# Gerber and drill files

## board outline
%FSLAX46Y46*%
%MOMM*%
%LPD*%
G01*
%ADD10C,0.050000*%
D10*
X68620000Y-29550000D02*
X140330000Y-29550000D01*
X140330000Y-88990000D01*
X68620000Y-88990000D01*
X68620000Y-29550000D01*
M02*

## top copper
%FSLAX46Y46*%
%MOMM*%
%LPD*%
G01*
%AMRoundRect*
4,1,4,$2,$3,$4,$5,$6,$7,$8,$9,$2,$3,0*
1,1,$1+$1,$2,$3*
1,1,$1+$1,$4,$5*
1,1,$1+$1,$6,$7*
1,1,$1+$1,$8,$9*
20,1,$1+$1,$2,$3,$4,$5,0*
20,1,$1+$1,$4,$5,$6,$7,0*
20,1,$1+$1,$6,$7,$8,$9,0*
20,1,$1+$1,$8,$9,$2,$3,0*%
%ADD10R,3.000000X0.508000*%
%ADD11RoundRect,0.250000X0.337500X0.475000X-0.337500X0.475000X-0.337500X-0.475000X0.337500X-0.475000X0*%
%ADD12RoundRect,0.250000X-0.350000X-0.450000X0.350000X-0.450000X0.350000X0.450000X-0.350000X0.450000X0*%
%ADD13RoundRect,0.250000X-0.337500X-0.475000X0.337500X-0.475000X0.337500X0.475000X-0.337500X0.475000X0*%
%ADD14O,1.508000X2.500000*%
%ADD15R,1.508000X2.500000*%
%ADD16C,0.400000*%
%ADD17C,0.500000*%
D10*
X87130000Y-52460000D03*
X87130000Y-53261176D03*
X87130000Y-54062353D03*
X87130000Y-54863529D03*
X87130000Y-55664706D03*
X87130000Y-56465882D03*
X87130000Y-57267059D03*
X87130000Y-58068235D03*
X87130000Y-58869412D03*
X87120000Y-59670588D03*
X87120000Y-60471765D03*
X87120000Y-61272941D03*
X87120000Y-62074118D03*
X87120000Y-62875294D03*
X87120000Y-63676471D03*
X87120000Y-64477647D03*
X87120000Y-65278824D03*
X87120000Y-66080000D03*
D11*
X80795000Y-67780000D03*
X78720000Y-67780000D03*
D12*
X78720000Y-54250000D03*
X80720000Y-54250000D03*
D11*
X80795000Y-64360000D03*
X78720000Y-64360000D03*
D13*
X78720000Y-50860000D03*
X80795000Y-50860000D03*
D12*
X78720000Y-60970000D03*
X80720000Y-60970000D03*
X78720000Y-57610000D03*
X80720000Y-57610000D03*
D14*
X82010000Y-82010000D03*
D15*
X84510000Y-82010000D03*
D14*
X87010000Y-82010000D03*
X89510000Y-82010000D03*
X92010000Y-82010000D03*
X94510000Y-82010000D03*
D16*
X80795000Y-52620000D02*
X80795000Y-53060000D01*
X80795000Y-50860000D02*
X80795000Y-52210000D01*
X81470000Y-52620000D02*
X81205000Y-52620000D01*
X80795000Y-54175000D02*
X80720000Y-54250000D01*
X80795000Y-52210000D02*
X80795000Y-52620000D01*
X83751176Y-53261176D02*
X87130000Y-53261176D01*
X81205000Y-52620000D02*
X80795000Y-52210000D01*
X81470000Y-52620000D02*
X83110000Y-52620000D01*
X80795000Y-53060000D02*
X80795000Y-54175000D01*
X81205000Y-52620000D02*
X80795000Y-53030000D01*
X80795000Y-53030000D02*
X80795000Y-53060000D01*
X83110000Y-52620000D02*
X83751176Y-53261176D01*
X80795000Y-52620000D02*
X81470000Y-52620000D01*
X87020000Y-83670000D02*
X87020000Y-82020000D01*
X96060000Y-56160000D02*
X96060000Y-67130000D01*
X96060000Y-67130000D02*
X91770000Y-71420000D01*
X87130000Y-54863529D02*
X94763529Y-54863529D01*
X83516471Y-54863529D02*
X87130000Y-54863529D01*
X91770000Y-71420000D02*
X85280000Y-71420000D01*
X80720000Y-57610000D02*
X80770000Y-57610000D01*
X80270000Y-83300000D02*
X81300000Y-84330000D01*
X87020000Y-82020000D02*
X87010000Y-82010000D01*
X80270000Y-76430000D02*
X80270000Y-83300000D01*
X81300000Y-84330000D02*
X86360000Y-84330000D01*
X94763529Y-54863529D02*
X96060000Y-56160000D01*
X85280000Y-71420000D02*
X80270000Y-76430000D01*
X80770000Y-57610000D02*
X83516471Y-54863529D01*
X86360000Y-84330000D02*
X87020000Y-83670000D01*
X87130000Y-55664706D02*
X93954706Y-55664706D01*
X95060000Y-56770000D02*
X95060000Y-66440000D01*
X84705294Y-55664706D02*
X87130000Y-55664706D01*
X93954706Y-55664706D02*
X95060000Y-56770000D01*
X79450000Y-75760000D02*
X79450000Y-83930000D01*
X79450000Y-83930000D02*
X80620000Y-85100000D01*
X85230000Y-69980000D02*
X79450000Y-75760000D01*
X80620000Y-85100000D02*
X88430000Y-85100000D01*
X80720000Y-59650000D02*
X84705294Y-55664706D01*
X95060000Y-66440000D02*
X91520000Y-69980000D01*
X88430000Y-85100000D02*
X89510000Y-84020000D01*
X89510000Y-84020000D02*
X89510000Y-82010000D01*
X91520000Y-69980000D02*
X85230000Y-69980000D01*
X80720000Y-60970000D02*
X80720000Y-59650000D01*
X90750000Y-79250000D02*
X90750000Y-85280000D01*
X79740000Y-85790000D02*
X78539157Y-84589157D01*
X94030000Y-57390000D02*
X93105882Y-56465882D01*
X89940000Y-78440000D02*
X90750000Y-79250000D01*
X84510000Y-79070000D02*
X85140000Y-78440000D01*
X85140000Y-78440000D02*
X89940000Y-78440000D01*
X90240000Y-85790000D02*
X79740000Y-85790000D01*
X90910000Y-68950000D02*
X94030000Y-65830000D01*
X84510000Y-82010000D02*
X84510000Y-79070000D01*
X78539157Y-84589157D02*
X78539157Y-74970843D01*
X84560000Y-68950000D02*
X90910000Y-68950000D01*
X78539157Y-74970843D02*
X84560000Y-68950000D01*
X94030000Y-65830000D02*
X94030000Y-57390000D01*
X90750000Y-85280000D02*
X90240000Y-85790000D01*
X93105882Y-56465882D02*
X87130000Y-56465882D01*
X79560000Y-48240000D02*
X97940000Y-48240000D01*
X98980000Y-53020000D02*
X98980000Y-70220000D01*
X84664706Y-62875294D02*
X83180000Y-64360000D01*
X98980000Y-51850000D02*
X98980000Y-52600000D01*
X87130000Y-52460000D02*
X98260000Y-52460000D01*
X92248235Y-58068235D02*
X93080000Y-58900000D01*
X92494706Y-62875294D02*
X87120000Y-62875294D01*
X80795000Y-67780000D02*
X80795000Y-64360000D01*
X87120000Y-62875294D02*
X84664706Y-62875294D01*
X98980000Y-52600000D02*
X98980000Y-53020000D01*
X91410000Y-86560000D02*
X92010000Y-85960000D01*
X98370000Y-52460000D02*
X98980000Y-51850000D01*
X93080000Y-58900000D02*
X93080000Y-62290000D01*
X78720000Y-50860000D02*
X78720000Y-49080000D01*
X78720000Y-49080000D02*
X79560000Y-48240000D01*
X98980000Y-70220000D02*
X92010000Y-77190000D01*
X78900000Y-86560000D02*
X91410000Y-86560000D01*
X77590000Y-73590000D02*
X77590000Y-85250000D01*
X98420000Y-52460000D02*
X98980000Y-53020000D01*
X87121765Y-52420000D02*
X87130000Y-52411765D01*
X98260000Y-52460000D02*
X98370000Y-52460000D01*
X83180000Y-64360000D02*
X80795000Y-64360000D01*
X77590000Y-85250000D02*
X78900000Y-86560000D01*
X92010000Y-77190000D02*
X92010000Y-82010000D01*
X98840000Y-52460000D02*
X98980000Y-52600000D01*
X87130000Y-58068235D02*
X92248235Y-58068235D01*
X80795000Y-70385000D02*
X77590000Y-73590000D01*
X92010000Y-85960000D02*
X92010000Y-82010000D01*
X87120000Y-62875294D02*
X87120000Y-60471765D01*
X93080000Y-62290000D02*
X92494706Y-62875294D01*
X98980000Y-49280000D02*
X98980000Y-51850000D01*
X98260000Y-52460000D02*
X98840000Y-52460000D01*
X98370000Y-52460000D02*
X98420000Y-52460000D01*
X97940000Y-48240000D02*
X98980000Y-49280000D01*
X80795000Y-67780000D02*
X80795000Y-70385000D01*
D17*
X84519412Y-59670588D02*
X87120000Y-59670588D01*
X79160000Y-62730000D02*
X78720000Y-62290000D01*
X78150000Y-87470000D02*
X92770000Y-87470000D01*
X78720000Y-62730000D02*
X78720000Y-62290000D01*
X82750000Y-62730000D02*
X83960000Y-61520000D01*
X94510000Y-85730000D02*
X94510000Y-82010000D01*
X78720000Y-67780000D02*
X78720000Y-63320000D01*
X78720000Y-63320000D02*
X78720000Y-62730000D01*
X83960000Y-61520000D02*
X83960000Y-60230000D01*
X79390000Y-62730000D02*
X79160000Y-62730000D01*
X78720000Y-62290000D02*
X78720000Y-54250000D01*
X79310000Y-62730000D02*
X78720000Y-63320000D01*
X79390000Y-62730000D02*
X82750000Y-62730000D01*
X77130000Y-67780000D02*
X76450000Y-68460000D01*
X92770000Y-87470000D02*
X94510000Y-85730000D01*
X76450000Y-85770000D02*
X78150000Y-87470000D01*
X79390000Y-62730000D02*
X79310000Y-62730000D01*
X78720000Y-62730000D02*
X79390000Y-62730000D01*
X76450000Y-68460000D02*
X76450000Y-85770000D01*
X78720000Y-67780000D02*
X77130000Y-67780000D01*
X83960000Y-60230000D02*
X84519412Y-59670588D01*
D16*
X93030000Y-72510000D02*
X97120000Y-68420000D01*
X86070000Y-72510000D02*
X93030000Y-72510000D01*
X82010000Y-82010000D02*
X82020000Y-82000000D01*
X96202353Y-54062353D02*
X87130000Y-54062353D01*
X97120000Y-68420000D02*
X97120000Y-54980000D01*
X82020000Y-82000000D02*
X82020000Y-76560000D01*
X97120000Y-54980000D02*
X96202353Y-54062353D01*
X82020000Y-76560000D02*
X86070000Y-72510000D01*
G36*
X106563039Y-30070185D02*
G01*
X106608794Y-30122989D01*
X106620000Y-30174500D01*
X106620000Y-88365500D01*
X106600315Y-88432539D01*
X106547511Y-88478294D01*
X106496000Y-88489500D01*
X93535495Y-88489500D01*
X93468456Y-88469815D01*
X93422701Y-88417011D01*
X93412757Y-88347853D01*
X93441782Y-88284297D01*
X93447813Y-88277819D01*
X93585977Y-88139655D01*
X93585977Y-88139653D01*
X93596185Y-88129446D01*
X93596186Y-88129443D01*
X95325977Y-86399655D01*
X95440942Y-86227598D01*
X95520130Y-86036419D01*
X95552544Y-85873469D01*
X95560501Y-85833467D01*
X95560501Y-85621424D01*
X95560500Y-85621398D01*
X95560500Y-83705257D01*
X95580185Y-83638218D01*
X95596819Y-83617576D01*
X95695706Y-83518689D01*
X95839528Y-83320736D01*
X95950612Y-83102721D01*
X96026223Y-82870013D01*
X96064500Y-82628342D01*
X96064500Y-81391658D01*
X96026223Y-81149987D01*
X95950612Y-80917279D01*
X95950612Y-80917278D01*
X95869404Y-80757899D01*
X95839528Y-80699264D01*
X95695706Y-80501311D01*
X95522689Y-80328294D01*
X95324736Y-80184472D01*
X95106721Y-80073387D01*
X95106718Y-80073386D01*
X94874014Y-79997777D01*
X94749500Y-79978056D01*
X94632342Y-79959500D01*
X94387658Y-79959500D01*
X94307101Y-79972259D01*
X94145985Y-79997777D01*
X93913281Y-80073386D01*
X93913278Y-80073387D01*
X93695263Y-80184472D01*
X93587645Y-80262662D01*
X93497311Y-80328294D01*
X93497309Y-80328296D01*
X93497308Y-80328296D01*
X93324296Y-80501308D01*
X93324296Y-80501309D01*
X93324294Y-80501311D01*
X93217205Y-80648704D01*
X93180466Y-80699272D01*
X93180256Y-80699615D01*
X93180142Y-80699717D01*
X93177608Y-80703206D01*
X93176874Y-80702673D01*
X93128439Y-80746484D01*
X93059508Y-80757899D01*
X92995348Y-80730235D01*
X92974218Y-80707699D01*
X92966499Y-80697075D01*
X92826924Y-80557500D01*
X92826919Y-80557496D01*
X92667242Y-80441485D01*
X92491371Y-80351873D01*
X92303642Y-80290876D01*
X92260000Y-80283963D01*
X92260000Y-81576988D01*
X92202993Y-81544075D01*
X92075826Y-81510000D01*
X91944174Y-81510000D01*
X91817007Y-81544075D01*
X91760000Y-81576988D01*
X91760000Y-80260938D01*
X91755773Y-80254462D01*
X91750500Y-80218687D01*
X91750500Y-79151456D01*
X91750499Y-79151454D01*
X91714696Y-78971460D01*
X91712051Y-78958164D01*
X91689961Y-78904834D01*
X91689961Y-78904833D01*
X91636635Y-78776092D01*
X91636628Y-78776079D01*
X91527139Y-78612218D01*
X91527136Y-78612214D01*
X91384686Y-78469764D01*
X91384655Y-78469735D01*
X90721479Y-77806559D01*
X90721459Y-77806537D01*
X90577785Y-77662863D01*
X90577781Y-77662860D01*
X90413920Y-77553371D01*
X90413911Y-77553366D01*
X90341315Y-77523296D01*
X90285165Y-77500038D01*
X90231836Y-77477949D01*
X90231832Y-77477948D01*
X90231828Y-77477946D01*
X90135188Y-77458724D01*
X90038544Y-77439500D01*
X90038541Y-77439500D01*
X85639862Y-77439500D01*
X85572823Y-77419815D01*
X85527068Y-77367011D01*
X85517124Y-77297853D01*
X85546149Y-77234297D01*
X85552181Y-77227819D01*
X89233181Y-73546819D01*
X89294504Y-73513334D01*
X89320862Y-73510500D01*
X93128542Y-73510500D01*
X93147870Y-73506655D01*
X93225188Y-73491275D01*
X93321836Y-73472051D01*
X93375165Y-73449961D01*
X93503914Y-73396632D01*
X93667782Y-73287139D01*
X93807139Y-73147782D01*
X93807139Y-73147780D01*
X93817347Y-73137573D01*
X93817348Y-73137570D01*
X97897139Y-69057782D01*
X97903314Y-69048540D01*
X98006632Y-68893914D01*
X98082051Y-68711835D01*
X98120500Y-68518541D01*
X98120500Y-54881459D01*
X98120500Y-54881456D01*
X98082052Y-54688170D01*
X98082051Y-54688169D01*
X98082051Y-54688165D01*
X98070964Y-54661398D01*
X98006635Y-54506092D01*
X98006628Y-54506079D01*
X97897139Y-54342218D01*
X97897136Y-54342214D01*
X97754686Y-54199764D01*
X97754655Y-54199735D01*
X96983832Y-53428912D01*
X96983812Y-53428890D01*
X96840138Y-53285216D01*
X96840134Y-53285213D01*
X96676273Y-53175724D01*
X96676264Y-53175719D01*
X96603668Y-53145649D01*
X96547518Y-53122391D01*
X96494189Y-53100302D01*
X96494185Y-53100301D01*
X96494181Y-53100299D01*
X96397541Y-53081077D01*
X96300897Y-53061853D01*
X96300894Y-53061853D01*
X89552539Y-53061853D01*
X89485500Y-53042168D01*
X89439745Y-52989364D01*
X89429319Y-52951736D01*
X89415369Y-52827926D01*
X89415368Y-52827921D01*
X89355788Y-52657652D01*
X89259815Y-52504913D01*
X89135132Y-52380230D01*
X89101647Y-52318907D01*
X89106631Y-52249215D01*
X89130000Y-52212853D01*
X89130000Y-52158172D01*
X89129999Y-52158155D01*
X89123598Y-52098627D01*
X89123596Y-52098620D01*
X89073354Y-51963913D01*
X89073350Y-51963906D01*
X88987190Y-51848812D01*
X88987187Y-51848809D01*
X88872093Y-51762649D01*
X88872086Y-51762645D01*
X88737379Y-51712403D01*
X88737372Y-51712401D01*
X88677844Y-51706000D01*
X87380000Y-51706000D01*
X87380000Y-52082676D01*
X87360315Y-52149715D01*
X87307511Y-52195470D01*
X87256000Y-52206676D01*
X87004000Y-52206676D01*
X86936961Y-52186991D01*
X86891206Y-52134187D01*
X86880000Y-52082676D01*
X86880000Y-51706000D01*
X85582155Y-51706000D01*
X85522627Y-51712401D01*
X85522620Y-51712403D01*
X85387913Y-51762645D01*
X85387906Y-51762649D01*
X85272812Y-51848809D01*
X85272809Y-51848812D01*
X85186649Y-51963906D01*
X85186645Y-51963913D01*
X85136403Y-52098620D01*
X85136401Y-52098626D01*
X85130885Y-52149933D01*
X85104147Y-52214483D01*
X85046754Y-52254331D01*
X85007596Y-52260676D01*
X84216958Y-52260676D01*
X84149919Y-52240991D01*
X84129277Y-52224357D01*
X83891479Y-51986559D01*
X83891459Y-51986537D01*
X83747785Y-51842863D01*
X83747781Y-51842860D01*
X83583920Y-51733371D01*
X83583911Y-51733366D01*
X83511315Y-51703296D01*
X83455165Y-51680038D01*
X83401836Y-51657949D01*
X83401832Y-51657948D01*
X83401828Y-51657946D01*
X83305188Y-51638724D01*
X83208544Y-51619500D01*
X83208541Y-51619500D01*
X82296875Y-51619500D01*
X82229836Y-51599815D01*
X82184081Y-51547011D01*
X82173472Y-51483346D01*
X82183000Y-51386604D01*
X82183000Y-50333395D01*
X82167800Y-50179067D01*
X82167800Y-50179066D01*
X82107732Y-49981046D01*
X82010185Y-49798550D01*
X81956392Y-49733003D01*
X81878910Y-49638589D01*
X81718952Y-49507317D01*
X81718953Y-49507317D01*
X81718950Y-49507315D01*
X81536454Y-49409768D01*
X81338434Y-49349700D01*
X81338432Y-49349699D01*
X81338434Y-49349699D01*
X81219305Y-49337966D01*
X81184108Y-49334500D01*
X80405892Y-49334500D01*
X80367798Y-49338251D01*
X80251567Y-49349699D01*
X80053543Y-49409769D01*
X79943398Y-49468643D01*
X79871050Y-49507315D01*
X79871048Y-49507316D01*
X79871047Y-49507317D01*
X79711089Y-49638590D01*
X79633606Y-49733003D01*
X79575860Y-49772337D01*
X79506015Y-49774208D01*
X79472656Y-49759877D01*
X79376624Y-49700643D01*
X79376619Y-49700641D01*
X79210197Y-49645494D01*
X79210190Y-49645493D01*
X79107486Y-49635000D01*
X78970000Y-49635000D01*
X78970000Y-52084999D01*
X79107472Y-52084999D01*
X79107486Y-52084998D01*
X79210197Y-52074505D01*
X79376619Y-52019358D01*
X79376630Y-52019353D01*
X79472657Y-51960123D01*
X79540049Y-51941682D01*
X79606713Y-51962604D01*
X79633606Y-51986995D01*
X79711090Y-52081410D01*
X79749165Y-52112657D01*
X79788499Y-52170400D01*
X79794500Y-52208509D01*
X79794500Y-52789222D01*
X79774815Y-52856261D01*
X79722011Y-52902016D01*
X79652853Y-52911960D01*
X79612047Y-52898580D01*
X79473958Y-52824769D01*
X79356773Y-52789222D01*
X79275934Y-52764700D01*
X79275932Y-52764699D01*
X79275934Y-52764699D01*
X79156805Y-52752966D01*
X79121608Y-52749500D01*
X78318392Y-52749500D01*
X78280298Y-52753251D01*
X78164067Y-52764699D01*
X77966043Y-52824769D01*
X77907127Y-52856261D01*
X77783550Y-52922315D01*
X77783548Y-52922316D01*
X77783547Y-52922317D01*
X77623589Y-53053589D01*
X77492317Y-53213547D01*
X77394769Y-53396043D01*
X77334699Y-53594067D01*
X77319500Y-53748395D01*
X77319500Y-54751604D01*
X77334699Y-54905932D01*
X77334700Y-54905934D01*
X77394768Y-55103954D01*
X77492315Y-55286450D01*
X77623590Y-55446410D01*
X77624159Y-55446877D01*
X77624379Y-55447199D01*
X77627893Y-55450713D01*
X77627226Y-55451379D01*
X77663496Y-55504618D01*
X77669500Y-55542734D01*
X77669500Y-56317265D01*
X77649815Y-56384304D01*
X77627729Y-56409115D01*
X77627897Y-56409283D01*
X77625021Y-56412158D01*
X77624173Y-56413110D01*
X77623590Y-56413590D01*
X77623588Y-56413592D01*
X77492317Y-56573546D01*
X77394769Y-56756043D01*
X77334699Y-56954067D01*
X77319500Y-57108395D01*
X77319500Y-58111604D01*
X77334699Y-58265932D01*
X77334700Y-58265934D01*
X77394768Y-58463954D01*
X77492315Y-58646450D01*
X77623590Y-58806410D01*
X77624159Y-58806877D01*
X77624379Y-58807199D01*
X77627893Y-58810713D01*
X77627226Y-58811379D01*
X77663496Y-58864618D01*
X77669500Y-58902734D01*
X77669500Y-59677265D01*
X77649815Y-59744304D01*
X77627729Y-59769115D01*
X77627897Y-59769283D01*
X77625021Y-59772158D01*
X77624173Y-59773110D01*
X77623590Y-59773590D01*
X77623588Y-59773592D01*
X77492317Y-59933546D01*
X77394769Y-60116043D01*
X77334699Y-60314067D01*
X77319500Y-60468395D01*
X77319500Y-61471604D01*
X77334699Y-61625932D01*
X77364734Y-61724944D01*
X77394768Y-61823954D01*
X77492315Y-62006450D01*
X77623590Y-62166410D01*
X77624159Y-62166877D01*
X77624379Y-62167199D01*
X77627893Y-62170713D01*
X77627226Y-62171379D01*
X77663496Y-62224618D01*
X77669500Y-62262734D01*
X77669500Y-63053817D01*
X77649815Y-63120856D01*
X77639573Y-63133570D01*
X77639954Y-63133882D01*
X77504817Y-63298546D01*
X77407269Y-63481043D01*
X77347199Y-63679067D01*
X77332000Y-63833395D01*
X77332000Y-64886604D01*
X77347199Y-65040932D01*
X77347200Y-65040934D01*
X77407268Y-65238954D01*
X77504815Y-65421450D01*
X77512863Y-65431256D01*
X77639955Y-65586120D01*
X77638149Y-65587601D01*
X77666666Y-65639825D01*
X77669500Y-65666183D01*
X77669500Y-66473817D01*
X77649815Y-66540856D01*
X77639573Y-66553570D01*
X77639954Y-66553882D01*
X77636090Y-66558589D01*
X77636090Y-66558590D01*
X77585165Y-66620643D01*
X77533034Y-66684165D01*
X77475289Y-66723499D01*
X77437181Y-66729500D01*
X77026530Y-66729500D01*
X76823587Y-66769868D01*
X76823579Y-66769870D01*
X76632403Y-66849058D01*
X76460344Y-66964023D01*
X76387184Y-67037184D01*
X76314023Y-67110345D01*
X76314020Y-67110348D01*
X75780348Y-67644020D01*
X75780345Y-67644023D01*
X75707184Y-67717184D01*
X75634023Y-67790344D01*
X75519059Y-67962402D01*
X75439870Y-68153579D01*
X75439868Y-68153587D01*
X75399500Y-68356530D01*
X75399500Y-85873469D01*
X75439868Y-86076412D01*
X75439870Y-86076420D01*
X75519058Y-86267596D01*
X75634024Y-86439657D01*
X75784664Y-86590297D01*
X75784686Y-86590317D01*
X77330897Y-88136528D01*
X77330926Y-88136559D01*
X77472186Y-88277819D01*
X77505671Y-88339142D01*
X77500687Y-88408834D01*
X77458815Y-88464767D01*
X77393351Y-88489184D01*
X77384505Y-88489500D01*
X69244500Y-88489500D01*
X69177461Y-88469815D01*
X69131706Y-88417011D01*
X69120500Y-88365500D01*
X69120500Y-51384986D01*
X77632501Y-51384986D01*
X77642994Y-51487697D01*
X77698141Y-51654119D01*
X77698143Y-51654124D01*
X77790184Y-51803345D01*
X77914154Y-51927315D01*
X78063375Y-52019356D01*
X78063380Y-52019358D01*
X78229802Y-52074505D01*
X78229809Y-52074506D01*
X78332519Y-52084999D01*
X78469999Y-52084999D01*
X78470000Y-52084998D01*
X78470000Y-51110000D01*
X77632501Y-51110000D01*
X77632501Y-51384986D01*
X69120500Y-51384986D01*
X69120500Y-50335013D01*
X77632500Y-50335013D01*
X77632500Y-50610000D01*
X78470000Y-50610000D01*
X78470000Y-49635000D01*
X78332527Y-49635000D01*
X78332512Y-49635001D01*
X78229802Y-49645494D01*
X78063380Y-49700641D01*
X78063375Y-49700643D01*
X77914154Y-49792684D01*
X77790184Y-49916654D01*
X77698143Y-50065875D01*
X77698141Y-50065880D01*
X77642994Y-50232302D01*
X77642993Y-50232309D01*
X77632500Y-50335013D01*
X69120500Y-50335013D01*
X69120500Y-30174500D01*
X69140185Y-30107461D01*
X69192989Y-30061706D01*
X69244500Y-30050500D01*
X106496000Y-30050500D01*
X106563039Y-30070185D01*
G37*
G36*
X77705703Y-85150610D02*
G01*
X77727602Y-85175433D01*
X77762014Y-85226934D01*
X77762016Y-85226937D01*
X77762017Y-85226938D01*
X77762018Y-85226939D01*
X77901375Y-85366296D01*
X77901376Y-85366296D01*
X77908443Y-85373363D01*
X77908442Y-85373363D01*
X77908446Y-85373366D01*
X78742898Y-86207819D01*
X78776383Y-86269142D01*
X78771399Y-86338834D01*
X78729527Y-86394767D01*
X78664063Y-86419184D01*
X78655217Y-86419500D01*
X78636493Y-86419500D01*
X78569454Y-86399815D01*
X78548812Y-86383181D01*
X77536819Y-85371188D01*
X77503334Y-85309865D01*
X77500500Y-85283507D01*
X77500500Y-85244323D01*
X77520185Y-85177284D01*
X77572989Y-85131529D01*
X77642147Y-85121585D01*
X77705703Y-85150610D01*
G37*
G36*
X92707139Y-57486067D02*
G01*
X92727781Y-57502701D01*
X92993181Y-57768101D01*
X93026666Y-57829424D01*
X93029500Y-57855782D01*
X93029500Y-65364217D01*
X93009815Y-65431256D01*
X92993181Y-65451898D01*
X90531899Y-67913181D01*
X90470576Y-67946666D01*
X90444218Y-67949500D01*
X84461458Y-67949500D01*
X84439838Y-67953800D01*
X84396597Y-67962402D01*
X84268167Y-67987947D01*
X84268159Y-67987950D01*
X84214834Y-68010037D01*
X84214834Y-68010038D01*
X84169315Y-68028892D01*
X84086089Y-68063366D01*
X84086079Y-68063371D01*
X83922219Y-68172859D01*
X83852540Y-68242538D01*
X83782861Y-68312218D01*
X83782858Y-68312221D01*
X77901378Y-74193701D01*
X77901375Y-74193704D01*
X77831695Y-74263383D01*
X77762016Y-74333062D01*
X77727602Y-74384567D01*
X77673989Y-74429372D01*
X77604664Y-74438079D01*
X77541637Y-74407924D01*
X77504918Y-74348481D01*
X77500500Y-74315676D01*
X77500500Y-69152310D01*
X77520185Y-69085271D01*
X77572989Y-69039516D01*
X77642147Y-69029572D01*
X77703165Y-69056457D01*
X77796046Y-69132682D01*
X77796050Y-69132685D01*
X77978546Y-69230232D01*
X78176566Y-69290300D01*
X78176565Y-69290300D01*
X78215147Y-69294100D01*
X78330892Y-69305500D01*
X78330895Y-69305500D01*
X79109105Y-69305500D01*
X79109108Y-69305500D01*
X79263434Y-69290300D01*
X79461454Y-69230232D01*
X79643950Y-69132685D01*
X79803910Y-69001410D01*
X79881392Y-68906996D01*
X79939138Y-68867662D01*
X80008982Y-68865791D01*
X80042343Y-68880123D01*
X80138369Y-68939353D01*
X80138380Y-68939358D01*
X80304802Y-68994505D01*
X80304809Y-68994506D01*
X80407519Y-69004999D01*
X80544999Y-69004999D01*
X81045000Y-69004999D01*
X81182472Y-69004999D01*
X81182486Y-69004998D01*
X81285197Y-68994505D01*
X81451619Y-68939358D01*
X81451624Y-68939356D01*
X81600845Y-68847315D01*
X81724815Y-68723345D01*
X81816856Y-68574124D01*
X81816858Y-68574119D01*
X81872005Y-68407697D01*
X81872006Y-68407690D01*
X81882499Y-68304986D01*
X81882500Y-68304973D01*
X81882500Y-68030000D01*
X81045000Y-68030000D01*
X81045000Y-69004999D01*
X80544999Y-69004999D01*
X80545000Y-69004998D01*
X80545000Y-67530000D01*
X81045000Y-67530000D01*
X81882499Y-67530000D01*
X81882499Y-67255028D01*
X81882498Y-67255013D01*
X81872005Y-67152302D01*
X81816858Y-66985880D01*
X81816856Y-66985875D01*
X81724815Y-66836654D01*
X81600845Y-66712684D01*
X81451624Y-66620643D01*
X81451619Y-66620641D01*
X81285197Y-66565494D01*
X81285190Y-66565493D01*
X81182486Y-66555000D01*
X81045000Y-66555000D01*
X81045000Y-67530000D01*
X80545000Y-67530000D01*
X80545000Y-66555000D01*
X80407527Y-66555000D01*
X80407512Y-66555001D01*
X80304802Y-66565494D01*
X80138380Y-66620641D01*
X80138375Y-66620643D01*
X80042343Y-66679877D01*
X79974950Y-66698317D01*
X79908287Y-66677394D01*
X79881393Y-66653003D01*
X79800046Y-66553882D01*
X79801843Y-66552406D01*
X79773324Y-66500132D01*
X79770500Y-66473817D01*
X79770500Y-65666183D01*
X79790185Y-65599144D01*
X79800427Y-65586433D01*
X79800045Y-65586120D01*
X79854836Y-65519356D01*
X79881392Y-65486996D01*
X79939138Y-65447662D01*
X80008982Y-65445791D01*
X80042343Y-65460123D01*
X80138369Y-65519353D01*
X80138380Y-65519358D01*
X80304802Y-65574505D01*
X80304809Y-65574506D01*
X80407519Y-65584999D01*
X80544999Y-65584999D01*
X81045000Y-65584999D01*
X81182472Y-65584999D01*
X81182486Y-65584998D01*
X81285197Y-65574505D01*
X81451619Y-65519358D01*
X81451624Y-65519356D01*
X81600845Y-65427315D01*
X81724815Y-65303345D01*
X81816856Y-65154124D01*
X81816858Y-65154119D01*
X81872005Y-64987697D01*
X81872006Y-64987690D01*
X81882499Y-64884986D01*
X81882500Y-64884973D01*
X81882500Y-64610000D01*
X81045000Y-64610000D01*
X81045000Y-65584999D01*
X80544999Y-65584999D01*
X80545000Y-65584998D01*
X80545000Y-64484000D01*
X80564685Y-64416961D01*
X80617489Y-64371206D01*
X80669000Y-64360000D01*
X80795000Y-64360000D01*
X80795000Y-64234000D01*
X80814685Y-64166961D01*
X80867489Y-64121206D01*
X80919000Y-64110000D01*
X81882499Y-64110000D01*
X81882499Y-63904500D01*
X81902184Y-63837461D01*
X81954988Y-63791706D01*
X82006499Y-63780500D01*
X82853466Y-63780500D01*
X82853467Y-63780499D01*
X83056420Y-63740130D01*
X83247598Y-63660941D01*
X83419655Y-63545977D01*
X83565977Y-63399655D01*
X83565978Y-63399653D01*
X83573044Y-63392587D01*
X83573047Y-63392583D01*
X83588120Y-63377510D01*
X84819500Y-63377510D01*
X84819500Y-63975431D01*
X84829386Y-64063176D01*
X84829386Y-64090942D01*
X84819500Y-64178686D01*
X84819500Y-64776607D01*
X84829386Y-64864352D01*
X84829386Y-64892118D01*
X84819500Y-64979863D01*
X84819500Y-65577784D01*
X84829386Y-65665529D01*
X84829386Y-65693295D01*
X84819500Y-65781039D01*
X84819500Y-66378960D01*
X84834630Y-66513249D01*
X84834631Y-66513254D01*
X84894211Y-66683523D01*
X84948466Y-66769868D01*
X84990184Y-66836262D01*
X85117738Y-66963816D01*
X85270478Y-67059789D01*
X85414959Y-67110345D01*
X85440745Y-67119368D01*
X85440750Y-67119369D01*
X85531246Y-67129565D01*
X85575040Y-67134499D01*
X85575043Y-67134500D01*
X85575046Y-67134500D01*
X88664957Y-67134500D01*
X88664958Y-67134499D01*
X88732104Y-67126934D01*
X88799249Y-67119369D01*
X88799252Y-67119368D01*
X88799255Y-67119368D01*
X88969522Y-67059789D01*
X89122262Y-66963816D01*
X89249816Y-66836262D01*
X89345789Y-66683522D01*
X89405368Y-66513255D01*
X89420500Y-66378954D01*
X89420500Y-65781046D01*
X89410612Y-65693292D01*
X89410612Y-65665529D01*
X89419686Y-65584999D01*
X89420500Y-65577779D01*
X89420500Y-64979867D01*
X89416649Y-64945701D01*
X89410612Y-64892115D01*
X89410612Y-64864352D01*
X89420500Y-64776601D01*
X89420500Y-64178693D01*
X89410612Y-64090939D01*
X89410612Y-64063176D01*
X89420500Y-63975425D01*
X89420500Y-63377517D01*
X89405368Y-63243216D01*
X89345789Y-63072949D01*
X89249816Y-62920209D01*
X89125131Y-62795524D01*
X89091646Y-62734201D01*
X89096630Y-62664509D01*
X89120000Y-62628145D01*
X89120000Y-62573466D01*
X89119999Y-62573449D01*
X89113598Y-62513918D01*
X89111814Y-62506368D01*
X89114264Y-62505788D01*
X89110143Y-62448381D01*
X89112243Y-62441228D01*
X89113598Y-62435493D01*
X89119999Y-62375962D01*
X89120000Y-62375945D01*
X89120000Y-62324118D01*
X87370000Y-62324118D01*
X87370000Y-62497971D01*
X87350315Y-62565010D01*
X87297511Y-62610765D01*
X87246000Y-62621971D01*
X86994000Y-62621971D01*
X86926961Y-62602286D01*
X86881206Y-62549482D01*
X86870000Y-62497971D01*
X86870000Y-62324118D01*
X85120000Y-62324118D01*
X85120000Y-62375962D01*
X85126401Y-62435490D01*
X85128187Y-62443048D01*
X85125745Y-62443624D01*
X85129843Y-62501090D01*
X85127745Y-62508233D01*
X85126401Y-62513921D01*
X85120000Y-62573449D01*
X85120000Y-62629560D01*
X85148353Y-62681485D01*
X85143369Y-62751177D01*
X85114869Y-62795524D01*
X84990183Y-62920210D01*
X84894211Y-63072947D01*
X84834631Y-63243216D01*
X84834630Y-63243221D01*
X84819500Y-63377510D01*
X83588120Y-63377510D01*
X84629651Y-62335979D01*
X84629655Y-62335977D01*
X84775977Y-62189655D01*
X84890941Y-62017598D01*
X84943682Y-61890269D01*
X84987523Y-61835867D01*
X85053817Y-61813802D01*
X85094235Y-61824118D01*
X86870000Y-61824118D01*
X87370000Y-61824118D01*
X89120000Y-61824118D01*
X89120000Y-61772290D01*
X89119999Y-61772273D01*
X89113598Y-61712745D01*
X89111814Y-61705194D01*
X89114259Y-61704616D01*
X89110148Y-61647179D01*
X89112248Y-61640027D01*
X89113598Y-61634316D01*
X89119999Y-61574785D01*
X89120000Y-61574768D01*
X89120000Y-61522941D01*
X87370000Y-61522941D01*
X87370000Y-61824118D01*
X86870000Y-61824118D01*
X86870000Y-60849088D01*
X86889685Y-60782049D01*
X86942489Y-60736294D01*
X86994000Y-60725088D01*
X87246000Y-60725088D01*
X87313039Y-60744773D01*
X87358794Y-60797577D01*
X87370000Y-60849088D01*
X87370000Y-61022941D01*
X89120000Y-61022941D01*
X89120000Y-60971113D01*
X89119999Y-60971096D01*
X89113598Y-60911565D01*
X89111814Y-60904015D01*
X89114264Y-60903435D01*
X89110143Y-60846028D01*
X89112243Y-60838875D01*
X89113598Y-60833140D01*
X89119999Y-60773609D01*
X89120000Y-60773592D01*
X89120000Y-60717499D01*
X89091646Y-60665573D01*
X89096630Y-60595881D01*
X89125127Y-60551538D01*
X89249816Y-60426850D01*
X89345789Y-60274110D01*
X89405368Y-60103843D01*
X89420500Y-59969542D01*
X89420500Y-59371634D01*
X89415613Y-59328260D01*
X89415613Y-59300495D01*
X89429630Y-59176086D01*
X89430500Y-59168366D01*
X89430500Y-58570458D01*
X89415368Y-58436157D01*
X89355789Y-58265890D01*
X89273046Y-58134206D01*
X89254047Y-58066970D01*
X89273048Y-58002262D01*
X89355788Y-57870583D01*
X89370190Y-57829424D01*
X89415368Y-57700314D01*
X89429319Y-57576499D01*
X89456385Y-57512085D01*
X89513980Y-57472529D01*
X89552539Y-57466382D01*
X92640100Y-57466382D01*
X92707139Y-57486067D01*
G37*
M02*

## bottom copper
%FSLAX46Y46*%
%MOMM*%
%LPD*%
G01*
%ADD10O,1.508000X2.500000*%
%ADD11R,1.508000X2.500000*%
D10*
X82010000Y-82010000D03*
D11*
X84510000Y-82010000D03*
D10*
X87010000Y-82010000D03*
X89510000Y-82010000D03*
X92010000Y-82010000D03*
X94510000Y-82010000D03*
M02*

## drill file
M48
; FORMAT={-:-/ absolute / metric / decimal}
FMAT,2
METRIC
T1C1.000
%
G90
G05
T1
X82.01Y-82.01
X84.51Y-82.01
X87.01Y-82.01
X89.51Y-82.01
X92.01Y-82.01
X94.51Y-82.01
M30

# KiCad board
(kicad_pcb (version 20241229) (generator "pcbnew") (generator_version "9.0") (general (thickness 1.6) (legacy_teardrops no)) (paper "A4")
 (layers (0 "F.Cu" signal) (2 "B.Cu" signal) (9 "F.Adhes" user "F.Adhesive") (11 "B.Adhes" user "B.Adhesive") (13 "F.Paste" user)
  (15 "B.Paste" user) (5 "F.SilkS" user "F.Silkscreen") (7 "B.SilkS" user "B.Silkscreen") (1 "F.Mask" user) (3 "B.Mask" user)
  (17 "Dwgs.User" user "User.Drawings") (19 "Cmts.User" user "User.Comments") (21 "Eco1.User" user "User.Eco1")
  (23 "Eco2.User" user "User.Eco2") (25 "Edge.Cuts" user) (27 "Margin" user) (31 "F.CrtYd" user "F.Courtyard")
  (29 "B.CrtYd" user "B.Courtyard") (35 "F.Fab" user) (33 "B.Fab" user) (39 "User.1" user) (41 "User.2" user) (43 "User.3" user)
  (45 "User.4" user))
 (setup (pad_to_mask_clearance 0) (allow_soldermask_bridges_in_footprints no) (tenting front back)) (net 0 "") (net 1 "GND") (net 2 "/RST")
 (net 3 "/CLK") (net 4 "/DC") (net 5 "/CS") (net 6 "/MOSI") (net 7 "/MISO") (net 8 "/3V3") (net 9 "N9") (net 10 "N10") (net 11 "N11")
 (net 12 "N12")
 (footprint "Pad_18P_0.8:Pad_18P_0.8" (layer "F.Cu") (at 83.19 58.381176 -90)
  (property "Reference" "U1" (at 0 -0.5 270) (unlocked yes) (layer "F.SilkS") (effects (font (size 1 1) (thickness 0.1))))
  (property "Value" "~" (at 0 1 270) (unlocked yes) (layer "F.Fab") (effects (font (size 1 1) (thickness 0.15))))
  (pad "01" smd rect (at -5.921176 -3.94 270) (size 0.508 3) (layers "F.Cu" "F.Mask" "F.Paste") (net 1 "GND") (solder_mask_margin 0.102))
  (pad "02" smd rect (at -5.12 -3.94 270) (size 0.508 3) (layers "F.Cu" "F.Mask" "F.Paste") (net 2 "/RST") (solder_mask_margin 0.102))
  (pad "03" smd rect (at -4.318823 -3.94 270) (size 0.508 3) (layers "F.Cu" "F.Mask" "F.Paste") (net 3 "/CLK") (solder_mask_margin 0.102))
  (pad "04" smd rect (at -3.517647 -3.94 270) (size 0.508 3) (layers "F.Cu" "F.Mask" "F.Paste") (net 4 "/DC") (solder_mask_margin 0.102))
  (pad "05" smd rect (at -2.71647 -3.94 270) (size 0.508 3) (layers "F.Cu" "F.Mask" "F.Paste") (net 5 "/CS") (solder_mask_margin 0.102))
  (pad "06" smd rect (at -1.915294 -3.94 270) (size 0.508 3) (layers "F.Cu" "F.Mask" "F.Paste") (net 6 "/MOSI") (solder_mask_margin 0.102))
  (pad "07" smd rect (at -1.114117 -3.94 270) (size 0.508 3) (layers "F.Cu" "F.Mask" "F.Paste") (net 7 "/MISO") (solder_mask_margin 0.102))
  (pad "08" smd rect (at -0.312941 -3.94 270) (size 0.508 3) (layers "F.Cu" "F.Mask" "F.Paste") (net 1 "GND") (solder_mask_margin 0.102))
  (pad "09" smd rect (at 0.488236 -3.94 270) (size 0.508 3) (layers "F.Cu" "F.Mask" "F.Paste") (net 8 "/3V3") (solder_mask_margin 0.102))
  (pad "10" smd rect (at 1.289412 -3.93 270) (size 0.508 3) (layers "F.Cu" "F.Mask" "F.Paste") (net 8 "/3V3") (solder_mask_margin 0.102))
  (pad "11" smd rect (at 2.090589 -3.93 270) (size 0.508 3) (layers "F.Cu" "F.Mask" "F.Paste") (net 1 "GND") (solder_mask_margin 0.102))
  (pad "12" smd rect (at 2.891765 -3.93 270) (size 0.508 3) (layers "F.Cu" "F.Mask" "F.Paste") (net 1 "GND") (solder_mask_margin 0.102))
  (pad "13" smd rect (at 3.692942 -3.93 270) (size 0.508 3) (layers "F.Cu" "F.Mask" "F.Paste") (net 1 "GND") (solder_mask_margin 0.102))
  (pad "14" smd rect (at 4.494118 -3.93 270) (size 0.508 3) (layers "F.Cu" "F.Mask" "F.Paste") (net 1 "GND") (solder_mask_margin 0.102))
  (pad "15" smd rect (at 5.295295 -3.93 270) (size 0.508 3) (layers "F.Cu" "F.Mask" "F.Paste") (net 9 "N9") (solder_mask_margin 0.102))
  (pad "16" smd rect (at 6.096471 -3.93 270) (size 0.508 3) (layers "F.Cu" "F.Mask" "F.Paste") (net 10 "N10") (solder_mask_margin 0.102))
  (pad "17" smd rect (at 6.897648 -3.93 270) (size 0.508 3) (layers "F.Cu" "F.Mask" "F.Paste") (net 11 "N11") (solder_mask_margin 0.102))
  (pad "18" smd rect (at 7.698824 -3.93 270) (size 0.508 3) (layers "F.Cu" "F.Mask" "F.Paste") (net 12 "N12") (solder_mask_margin 0.102)))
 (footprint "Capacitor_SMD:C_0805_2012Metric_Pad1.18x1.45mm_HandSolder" (layer "F.Cu") (at 79.7575 67.78 180)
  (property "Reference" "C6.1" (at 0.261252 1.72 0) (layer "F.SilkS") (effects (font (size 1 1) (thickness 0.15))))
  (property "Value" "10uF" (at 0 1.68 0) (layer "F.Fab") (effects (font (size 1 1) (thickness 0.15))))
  (pad "1" smd roundrect (at -1.0375 0 180) (size 1.175 1.45) (layers "F.Cu" "F.Mask" "F.Paste") (roundrect_rratio 0.212766) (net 1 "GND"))
  (pad "2" smd roundrect (at 1.0375 0 180) (size 1.175 1.45) (layers "F.Cu" "F.Mask" "F.Paste") (roundrect_rratio 0.212766) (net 8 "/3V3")))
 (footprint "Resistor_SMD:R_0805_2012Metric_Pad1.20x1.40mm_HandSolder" (layer "F.Cu") (at 79.72 54.25)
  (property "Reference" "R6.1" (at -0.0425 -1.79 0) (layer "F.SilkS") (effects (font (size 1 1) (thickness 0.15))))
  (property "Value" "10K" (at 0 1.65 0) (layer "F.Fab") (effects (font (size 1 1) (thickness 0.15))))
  (pad "1" smd roundrect (at -1 0) (size 1.2 1.4) (layers "F.Cu" "F.Mask" "F.Paste") (roundrect_rratio 0.208333) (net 8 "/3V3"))
  (pad "2" smd roundrect (at 1 0) (size 1.2 1.4) (layers "F.Cu" "F.Mask" "F.Paste") (roundrect_rratio 0.208333) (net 2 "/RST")))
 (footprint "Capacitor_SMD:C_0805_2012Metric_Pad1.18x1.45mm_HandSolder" (layer "F.Cu") (at 79.7575 64.36 180)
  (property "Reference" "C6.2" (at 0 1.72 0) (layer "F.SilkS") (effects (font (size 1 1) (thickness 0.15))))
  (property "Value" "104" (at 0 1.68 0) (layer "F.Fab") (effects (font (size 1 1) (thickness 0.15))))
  (pad "1" smd roundrect (at -1.0375 0 180) (size 1.175 1.45) (layers "F.Cu" "F.Mask" "F.Paste") (roundrect_rratio 0.212766) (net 1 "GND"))
  (pad "2" smd roundrect (at 1.0375 0 180) (size 1.175 1.45) (layers "F.Cu" "F.Mask" "F.Paste") (roundrect_rratio 0.212766) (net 8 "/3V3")))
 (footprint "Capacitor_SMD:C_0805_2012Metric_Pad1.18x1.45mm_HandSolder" (layer "F.Cu") (at 79.7575 50.86)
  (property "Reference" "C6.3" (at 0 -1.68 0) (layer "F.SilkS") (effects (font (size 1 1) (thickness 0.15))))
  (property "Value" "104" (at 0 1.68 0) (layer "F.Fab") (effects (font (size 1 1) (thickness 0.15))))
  (pad "1" smd roundrect (at -1.0375 0) (size 1.175 1.45) (layers "F.Cu" "F.Mask" "F.Paste") (roundrect_rratio 0.212766) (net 1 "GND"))
  (pad "2" smd roundrect (at 1.0375 0) (size 1.175 1.45) (layers "F.Cu" "F.Mask" "F.Paste") (roundrect_rratio 0.212766) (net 2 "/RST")))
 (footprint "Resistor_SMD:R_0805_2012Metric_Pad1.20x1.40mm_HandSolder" (layer "F.Cu") (at 79.72 60.97)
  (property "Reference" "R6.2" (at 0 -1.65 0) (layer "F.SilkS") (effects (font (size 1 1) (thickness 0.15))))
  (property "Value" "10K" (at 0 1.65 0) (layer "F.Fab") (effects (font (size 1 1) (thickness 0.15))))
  (pad "1" smd roundrect (at -1 0) (size 1.2 1.4) (layers "F.Cu" "F.Mask" "F.Paste") (roundrect_rratio 0.208333) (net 8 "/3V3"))
  (pad "2" smd roundrect (at 1 0) (size 1.2 1.4) (layers "F.Cu" "F.Mask" "F.Paste") (roundrect_rratio 0.208333) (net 5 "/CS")))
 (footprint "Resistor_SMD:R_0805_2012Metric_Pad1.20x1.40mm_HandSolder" (layer "F.Cu") (at 79.72 57.61)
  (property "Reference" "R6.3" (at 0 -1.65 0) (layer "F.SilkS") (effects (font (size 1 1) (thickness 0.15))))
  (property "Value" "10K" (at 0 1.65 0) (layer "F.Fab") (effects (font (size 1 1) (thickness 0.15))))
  (pad "1" smd roundrect (at -1 0) (size 1.2 1.4) (layers "F.Cu" "F.Mask" "F.Paste") (roundrect_rratio 0.208333) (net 8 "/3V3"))
  (pad "2" smd roundrect (at 1 0) (size 1.2 1.4) (layers "F.Cu" "F.Mask" "F.Paste") (roundrect_rratio 0.208333) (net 4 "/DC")))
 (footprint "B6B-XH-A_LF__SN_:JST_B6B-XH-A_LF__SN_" (layer "B.Cu") (at 88.26 81.485 180)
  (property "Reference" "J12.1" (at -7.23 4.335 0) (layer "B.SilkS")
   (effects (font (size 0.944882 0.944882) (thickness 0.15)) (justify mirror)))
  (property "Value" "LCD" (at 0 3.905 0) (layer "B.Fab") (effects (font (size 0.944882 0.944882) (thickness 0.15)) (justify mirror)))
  (pad "1" thru_hole oval (at 6.25 -0.525 180) (size 1.508 2.5) (drill 1) (layers "*.Cu" "*.Mask") (remove_unused_layers no) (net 3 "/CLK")
   (solder_mask_margin 0.102))
  (pad "2" thru_hole rect (at 3.75 -0.525 180) (size 1.508 2.5) (drill 1) (layers "*.Cu" "*.Mask") (remove_unused_layers no) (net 6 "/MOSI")
   (solder_mask_margin 0.102))
  (pad "3" thru_hole oval (at 1.25 -0.525 180) (size 1.508 2.5) (drill 1) (layers "*.Cu" "*.Mask") (remove_unused_layers no) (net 4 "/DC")
   (solder_mask_margin 0.102))
  (pad "4" thru_hole oval (at -1.25 -0.525 180) (size 1.508 2.5) (drill 1) (layers "*.Cu" "*.Mask") (remove_unused_layers no) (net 5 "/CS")
   (solder_mask_margin 0.102))
  (pad "5" thru_hole oval (at -3.75 -0.525 180) (size 1.508 2.5) (drill 1) (layers "*.Cu" "*.Mask") (remove_unused_layers no) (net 1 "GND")
   (solder_mask_margin 0.102))
  (pad "6" thru_hole oval (at -6.25 -0.525 180) (size 1.508 2.5) (drill 1) (layers "*.Cu" "*.Mask") (remove_unused_layers no) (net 8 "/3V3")
   (solder_mask_margin 0.102)))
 (gr_rect (start 68.62 29.55) (end 140.33 88.99) (stroke (width 0.05) (type default)) (fill no) (layer "Edge.Cuts"))
 (segment (start 80.795 52.62) (end 80.795 53.06) (width 0.4) (layer "F.Cu") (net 2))
 (segment (start 80.795 50.86) (end 80.795 52.21) (width 0.4) (layer "F.Cu") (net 2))
 (segment (start 81.47 52.62) (end 81.205 52.62) (width 0.4) (layer "F.Cu") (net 2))
 (segment (start 80.795 54.175) (end 80.72 54.25) (width 0.4) (layer "F.Cu") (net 2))
 (segment (start 80.795 52.21) (end 80.795 52.62) (width 0.4) (layer "F.Cu") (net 2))
 (segment (start 83.751176 53.261176) (end 87.13 53.261176) (width 0.4) (layer "F.Cu") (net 2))
 (segment (start 81.205 52.62) (end 80.795 52.21) (width 0.4) (layer "F.Cu") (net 2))
 (segment (start 81.47 52.62) (end 83.11 52.62) (width 0.4) (layer "F.Cu") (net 2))
 (segment (start 80.795 53.06) (end 80.795 54.175) (width 0.4) (layer "F.Cu") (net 2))
 (segment (start 81.205 52.62) (end 80.795 53.03) (width 0.4) (layer "F.Cu") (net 2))
 (segment (start 80.795 53.03) (end 80.795 53.06) (width 0.4) (layer "F.Cu") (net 2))
 (segment (start 83.11 52.62) (end 83.751176 53.261176) (width 0.4) (layer "F.Cu") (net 2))
 (segment (start 80.795 52.62) (end 81.47 52.62) (width 0.4) (layer "F.Cu") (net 2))
 (segment (start 87.02 83.67) (end 87.02 82.02) (width 0.4) (layer "F.Cu") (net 4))
 (segment (start 96.06 56.16) (end 96.06 67.13) (width 0.4) (layer "F.Cu") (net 4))
 (segment (start 96.06 67.13) (end 91.77 71.42) (width 0.4) (layer "F.Cu") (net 4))
 (segment (start 87.13 54.863529) (end 94.763529 54.863529) (width 0.4) (layer "F.Cu") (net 4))
 (segment (start 83.516471 54.863529) (end 87.13 54.863529) (width 0.4) (layer "F.Cu") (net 4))
 (segment (start 91.77 71.42) (end 85.28 71.42) (width 0.4) (layer "F.Cu") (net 4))
 (segment (start 80.72 57.61) (end 80.77 57.61) (width 0.4) (layer "F.Cu") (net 4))
 (segment (start 80.27 83.3) (end 81.3 84.33) (width 0.4) (layer "F.Cu") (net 4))
 (segment (start 87.02 82.02) (end 87.01 82.01) (width 0.4) (layer "F.Cu") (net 4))
 (segment (start 80.27 76.43) (end 80.27 83.3) (width 0.4) (layer "F.Cu") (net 4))
 (segment (start 81.3 84.33) (end 86.36 84.33) (width 0.4) (layer "F.Cu") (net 4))
 (segment (start 94.763529 54.863529) (end 96.06 56.16) (width 0.4) (layer "F.Cu") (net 4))
 (segment (start 85.28 71.42) (end 80.27 76.43) (width 0.4) (layer "F.Cu") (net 4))
 (segment (start 80.77 57.61) (end 83.516471 54.863529) (width 0.4) (layer "F.Cu") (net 4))
 (segment (start 86.36 84.33) (end 87.02 83.67) (width 0.4) (layer "F.Cu") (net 4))
 (segment (start 87.13 55.664706) (end 93.954706 55.664706) (width 0.4) (layer "F.Cu") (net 5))
 (segment (start 95.06 56.77) (end 95.06 66.44) (width 0.4) (layer "F.Cu") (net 5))
 (segment (start 84.705294 55.664706) (end 87.13 55.664706) (width 0.4) (layer "F.Cu") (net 5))
 (segment (start 93.954706 55.664706) (end 95.06 56.77) (width 0.4) (layer "F.Cu") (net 5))
 (segment (start 79.45 75.76) (end 79.45 83.93) (width 0.4) (layer "F.Cu") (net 5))
 (segment (start 79.45 83.93) (end 80.62 85.1) (width 0.4) (layer "F.Cu") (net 5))
 (segment (start 85.23 69.98) (end 79.45 75.76) (width 0.4) (layer "F.Cu") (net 5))
 (segment (start 80.62 85.1) (end 88.43 85.1) (width 0.4) (layer "F.Cu") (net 5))
 (segment (start 80.72 59.65) (end 84.705294 55.664706) (width 0.4) (layer "F.Cu") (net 5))
 (segment (start 95.06 66.44) (end 91.52 69.98) (width 0.4) (layer "F.Cu") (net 5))
 (segment (start 88.43 85.1) (end 89.51 84.02) (width 0.4) (layer "F.Cu") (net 5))
 (segment (start 89.51 84.02) (end 89.51 82.01) (width 0.4) (layer "F.Cu") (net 5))
 (segment (start 91.52 69.98) (end 85.23 69.98) (width 0.4) (layer "F.Cu") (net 5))
 (segment (start 80.72 60.97) (end 80.72 59.65) (width 0.4) (layer "F.Cu") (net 5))
 (segment (start 90.75 79.25) (end 90.75 85.28) (width 0.4) (layer "F.Cu") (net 6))
 (segment (start 79.74 85.79) (end 78.539157 84.589157) (width 0.4) (layer "F.Cu") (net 6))
 (segment (start 94.03 57.39) (end 93.105882 56.465882) (width 0.4) (layer "F.Cu") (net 6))
 (segment (start 89.94 78.44) (end 90.75 79.25) (width 0.4) (layer "F.Cu") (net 6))
 (segment (start 84.51 79.07) (end 85.14 78.44) (width 0.4) (layer "F.Cu") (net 6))
 (segment (start 85.14 78.44) (end 89.94 78.44) (width 0.4) (layer "F.Cu") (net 6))
 (segment (start 90.24 85.79) (end 79.74 85.79) (width 0.4) (layer "F.Cu") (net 6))
 (segment (start 90.91 68.95) (end 94.03 65.83) (width 0.4) (layer "F.Cu") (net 6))
 (segment (start 84.51 82.01) (end 84.51 79.07) (width 0.4) (layer "F.Cu") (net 6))
 (segment (start 78.539157 84.589157) (end 78.539157 74.970843) (width 0.4) (layer "F.Cu") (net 6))
 (segment (start 84.56 68.95) (end 90.91 68.95) (width 0.4) (layer "F.Cu") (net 6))
 (segment (start 78.539157 74.970843) (end 84.56 68.95) (width 0.4) (layer "F.Cu") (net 6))
 (segment (start 94.03 65.83) (end 94.03 57.39) (width 0.4) (layer "F.Cu") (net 6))
 (segment (start 90.75 85.28) (end 90.24 85.79) (width 0.4) (layer "F.Cu") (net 6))
 (segment (start 93.105882 56.465882) (end 87.13 56.465882) (width 0.4) (layer "F.Cu") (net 6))
 (segment (start 79.56 48.24) (end 97.94 48.24) (width 0.4) (layer "F.Cu") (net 1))
 (segment (start 98.98 53.02) (end 98.98 70.22) (width 0.4) (layer "F.Cu") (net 1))
 (segment (start 84.664706 62.875294) (end 83.18 64.36) (width 0.4) (layer "F.Cu") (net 1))
 (segment (start 98.98 51.85) (end 98.98 52.6) (width 0.4) (layer "F.Cu") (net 1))
 (segment (start 87.13 52.46) (end 98.26 52.46) (width 0.4) (layer "F.Cu") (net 1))
 (segment (start 92.248235 58.068235) (end 93.08 58.9) (width 0.4) (layer "F.Cu") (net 1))
 (segment (start 92.494706 62.875294) (end 87.12 62.875294) (width 0.4) (layer "F.Cu") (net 1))
 (segment (start 80.795 67.78) (end 80.795 64.36) (width 0.4) (layer "F.Cu") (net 1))
 (segment (start 87.12 62.875294) (end 84.664706 62.875294) (width 0.4) (layer "F.Cu") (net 1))
 (segment (start 98.98 52.6) (end 98.98 53.02) (width 0.4) (layer "F.Cu") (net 1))
 (segment (start 91.41 86.56) (end 92.01 85.96) (width 0.4) (layer "F.Cu") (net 1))
 (segment (start 98.37 52.46) (end 98.98 51.85) (width 0.4) (layer "F.Cu") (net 1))
 (segment (start 93.08 58.9) (end 93.08 62.29) (width 0.4) (layer "F.Cu") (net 1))
 (segment (start 78.72 50.86) (end 78.72 49.08) (width 0.4) (layer "F.Cu") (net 1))
 (segment (start 78.72 49.08) (end 79.56 48.24) (width 0.4) (layer "F.Cu") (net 1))
 (segment (start 98.98 70.22) (end 92.01 77.19) (width 0.4) (layer "F.Cu") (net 1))
 (segment (start 78.9 86.56) (end 91.41 86.56) (width 0.4) (layer "F.Cu") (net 1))
 (segment (start 77.59 73.59) (end 77.59 85.25) (width 0.4) (layer "F.Cu") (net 1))
 (segment (start 98.42 52.46) (end 98.98 53.02) (width 0.4) (layer "F.Cu") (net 1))
 (segment (start 87.121765 52.42) (end 87.13 52.411765) (width 0.4) (layer "F.Cu") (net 1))
 (segment (start 98.26 52.46) (end 98.37 52.46) (width 0.4) (layer "F.Cu") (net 1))
 (segment (start 83.18 64.36) (end 80.795 64.36) (width 0.4) (layer "F.Cu") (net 1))
 (segment (start 77.59 85.25) (end 78.9 86.56) (width 0.4) (layer "F.Cu") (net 1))
 (segment (start 92.01 77.19) (end 92.01 82.01) (width 0.4) (layer "F.Cu") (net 1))
 (segment (start 98.84 52.46) (end 98.98 52.6) (width 0.4) (layer "F.Cu") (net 1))
 (segment (start 87.13 58.068235) (end 92.248235 58.068235) (width 0.4) (layer "F.Cu") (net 1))
 (segment (start 80.795 70.385) (end 77.59 73.59) (width 0.4) (layer "F.Cu") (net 1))
 (segment (start 92.01 85.96) (end 92.01 82.01) (width 0.4) (layer "F.Cu") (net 1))
 (segment (start 87.12 62.875294) (end 87.12 60.471765) (width 0.4) (layer "F.Cu") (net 1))
 (segment (start 93.08 62.29) (end 92.494706 62.875294) (width 0.4) (layer "F.Cu") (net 1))
 (segment (start 98.98 49.28) (end 98.98 51.85) (width 0.4) (layer "F.Cu") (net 1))
 (segment (start 98.26 52.46) (end 98.84 52.46) (width 0.4) (layer "F.Cu") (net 1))
 (segment (start 98.37 52.46) (end 98.42 52.46) (width 0.4) (layer "F.Cu") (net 1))
 (segment (start 97.94 48.24) (end 98.98 49.28) (width 0.4) (layer "F.Cu") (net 1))
 (segment (start 80.795 67.78) (end 80.795 70.385) (width 0.4) (layer "F.Cu") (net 1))
 (segment (start 84.519412 59.670588) (end 87.12 59.670588) (width 0.5) (layer "F.Cu") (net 8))
 (segment (start 79.16 62.73) (end 78.72 62.29) (width 0.5) (layer "F.Cu") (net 8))
 (segment (start 78.15 87.47) (end 92.77 87.47) (width 0.5) (layer "F.Cu") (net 8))
 (segment (start 78.72 62.73) (end 78.72 62.29) (width 0.5) (layer "F.Cu") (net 8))
 (segment (start 82.75 62.73) (end 83.96 61.52) (width 0.5) (layer "F.Cu") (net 8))
 (segment (start 94.51 85.73) (end 94.51 82.01) (width 0.5) (layer "F.Cu") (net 8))
 (segment (start 78.72 67.78) (end 78.72 63.32) (width 0.5) (layer "F.Cu") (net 8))
 (segment (start 78.72 63.32) (end 78.72 62.73) (width 0.5) (layer "F.Cu") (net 8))
 (segment (start 83.96 61.52) (end 83.96 60.23) (width 0.5) (layer "F.Cu") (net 8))
 (segment (start 79.39 62.73) (end 79.16 62.73) (width 0.5) (layer "F.Cu") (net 8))
 (segment (start 78.72 62.29) (end 78.72 54.25) (width 0.5) (layer "F.Cu") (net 8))
 (segment (start 79.31 62.73) (end 78.72 63.32) (width 0.5) (layer "F.Cu") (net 8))
 (segment (start 79.39 62.73) (end 82.75 62.73) (width 0.5) (layer "F.Cu") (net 8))
 (segment (start 77.13 67.78) (end 76.45 68.46) (width 0.5) (layer "F.Cu") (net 8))
 (segment (start 92.77 87.47) (end 94.51 85.73) (width 0.5) (layer "F.Cu") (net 8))
 (segment (start 76.45 85.77) (end 78.15 87.47) (width 0.5) (layer "F.Cu") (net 8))
 (segment (start 79.39 62.73) (end 79.31 62.73) (width 0.5) (layer "F.Cu") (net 8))
 (segment (start 78.72 62.73) (end 79.39 62.73) (width 0.5) (layer "F.Cu") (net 8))
 (segment (start 76.45 68.46) (end 76.45 85.77) (width 0.5) (layer "F.Cu") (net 8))
 (segment (start 78.72 67.78) (end 77.13 67.78) (width 0.5) (layer "F.Cu") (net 8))
 (segment (start 83.96 60.23) (end 84.519412 59.670588) (width 0.5) (layer "F.Cu") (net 8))
 (segment (start 93.03 72.51) (end 97.12 68.42) (width 0.4) (layer "F.Cu") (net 3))
 (segment (start 86.07 72.51) (end 93.03 72.51) (width 0.4) (layer "F.Cu") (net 3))
 (segment (start 82.01 82.01) (end 82.02 82) (width 0.4) (layer "F.Cu") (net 3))
 (segment (start 96.202353 54.062353) (end 87.13 54.062353) (width 0.4) (layer "F.Cu") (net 3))
 (segment (start 97.12 68.42) (end 97.12 54.98) (width 0.4) (layer "F.Cu") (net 3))
 (segment (start 82.02 82) (end 82.02 76.56) (width 0.4) (layer "F.Cu") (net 3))
 (segment (start 97.12 54.98) (end 96.202353 54.062353) (width 0.4) (layer "F.Cu") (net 3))
 (segment (start 82.02 76.56) (end 86.07 72.51) (width 0.4) (layer "F.Cu") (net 3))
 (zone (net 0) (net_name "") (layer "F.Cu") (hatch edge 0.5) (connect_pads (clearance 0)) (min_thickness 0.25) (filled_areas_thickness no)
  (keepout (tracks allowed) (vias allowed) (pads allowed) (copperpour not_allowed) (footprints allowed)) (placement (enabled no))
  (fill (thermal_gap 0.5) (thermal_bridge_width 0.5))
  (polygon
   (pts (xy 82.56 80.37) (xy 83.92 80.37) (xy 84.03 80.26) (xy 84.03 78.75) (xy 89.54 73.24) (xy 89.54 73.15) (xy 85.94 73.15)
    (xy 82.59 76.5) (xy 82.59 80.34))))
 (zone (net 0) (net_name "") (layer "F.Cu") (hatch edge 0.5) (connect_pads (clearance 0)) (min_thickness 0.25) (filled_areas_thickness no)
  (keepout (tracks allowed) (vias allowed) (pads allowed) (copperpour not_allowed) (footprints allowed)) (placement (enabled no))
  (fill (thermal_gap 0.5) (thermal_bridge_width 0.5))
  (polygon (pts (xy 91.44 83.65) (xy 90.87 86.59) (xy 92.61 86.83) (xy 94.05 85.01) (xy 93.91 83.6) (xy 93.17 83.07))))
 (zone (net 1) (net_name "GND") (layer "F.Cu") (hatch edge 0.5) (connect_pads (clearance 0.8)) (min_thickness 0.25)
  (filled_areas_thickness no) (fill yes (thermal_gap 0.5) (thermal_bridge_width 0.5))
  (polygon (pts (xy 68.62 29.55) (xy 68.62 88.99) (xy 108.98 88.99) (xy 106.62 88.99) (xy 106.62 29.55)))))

